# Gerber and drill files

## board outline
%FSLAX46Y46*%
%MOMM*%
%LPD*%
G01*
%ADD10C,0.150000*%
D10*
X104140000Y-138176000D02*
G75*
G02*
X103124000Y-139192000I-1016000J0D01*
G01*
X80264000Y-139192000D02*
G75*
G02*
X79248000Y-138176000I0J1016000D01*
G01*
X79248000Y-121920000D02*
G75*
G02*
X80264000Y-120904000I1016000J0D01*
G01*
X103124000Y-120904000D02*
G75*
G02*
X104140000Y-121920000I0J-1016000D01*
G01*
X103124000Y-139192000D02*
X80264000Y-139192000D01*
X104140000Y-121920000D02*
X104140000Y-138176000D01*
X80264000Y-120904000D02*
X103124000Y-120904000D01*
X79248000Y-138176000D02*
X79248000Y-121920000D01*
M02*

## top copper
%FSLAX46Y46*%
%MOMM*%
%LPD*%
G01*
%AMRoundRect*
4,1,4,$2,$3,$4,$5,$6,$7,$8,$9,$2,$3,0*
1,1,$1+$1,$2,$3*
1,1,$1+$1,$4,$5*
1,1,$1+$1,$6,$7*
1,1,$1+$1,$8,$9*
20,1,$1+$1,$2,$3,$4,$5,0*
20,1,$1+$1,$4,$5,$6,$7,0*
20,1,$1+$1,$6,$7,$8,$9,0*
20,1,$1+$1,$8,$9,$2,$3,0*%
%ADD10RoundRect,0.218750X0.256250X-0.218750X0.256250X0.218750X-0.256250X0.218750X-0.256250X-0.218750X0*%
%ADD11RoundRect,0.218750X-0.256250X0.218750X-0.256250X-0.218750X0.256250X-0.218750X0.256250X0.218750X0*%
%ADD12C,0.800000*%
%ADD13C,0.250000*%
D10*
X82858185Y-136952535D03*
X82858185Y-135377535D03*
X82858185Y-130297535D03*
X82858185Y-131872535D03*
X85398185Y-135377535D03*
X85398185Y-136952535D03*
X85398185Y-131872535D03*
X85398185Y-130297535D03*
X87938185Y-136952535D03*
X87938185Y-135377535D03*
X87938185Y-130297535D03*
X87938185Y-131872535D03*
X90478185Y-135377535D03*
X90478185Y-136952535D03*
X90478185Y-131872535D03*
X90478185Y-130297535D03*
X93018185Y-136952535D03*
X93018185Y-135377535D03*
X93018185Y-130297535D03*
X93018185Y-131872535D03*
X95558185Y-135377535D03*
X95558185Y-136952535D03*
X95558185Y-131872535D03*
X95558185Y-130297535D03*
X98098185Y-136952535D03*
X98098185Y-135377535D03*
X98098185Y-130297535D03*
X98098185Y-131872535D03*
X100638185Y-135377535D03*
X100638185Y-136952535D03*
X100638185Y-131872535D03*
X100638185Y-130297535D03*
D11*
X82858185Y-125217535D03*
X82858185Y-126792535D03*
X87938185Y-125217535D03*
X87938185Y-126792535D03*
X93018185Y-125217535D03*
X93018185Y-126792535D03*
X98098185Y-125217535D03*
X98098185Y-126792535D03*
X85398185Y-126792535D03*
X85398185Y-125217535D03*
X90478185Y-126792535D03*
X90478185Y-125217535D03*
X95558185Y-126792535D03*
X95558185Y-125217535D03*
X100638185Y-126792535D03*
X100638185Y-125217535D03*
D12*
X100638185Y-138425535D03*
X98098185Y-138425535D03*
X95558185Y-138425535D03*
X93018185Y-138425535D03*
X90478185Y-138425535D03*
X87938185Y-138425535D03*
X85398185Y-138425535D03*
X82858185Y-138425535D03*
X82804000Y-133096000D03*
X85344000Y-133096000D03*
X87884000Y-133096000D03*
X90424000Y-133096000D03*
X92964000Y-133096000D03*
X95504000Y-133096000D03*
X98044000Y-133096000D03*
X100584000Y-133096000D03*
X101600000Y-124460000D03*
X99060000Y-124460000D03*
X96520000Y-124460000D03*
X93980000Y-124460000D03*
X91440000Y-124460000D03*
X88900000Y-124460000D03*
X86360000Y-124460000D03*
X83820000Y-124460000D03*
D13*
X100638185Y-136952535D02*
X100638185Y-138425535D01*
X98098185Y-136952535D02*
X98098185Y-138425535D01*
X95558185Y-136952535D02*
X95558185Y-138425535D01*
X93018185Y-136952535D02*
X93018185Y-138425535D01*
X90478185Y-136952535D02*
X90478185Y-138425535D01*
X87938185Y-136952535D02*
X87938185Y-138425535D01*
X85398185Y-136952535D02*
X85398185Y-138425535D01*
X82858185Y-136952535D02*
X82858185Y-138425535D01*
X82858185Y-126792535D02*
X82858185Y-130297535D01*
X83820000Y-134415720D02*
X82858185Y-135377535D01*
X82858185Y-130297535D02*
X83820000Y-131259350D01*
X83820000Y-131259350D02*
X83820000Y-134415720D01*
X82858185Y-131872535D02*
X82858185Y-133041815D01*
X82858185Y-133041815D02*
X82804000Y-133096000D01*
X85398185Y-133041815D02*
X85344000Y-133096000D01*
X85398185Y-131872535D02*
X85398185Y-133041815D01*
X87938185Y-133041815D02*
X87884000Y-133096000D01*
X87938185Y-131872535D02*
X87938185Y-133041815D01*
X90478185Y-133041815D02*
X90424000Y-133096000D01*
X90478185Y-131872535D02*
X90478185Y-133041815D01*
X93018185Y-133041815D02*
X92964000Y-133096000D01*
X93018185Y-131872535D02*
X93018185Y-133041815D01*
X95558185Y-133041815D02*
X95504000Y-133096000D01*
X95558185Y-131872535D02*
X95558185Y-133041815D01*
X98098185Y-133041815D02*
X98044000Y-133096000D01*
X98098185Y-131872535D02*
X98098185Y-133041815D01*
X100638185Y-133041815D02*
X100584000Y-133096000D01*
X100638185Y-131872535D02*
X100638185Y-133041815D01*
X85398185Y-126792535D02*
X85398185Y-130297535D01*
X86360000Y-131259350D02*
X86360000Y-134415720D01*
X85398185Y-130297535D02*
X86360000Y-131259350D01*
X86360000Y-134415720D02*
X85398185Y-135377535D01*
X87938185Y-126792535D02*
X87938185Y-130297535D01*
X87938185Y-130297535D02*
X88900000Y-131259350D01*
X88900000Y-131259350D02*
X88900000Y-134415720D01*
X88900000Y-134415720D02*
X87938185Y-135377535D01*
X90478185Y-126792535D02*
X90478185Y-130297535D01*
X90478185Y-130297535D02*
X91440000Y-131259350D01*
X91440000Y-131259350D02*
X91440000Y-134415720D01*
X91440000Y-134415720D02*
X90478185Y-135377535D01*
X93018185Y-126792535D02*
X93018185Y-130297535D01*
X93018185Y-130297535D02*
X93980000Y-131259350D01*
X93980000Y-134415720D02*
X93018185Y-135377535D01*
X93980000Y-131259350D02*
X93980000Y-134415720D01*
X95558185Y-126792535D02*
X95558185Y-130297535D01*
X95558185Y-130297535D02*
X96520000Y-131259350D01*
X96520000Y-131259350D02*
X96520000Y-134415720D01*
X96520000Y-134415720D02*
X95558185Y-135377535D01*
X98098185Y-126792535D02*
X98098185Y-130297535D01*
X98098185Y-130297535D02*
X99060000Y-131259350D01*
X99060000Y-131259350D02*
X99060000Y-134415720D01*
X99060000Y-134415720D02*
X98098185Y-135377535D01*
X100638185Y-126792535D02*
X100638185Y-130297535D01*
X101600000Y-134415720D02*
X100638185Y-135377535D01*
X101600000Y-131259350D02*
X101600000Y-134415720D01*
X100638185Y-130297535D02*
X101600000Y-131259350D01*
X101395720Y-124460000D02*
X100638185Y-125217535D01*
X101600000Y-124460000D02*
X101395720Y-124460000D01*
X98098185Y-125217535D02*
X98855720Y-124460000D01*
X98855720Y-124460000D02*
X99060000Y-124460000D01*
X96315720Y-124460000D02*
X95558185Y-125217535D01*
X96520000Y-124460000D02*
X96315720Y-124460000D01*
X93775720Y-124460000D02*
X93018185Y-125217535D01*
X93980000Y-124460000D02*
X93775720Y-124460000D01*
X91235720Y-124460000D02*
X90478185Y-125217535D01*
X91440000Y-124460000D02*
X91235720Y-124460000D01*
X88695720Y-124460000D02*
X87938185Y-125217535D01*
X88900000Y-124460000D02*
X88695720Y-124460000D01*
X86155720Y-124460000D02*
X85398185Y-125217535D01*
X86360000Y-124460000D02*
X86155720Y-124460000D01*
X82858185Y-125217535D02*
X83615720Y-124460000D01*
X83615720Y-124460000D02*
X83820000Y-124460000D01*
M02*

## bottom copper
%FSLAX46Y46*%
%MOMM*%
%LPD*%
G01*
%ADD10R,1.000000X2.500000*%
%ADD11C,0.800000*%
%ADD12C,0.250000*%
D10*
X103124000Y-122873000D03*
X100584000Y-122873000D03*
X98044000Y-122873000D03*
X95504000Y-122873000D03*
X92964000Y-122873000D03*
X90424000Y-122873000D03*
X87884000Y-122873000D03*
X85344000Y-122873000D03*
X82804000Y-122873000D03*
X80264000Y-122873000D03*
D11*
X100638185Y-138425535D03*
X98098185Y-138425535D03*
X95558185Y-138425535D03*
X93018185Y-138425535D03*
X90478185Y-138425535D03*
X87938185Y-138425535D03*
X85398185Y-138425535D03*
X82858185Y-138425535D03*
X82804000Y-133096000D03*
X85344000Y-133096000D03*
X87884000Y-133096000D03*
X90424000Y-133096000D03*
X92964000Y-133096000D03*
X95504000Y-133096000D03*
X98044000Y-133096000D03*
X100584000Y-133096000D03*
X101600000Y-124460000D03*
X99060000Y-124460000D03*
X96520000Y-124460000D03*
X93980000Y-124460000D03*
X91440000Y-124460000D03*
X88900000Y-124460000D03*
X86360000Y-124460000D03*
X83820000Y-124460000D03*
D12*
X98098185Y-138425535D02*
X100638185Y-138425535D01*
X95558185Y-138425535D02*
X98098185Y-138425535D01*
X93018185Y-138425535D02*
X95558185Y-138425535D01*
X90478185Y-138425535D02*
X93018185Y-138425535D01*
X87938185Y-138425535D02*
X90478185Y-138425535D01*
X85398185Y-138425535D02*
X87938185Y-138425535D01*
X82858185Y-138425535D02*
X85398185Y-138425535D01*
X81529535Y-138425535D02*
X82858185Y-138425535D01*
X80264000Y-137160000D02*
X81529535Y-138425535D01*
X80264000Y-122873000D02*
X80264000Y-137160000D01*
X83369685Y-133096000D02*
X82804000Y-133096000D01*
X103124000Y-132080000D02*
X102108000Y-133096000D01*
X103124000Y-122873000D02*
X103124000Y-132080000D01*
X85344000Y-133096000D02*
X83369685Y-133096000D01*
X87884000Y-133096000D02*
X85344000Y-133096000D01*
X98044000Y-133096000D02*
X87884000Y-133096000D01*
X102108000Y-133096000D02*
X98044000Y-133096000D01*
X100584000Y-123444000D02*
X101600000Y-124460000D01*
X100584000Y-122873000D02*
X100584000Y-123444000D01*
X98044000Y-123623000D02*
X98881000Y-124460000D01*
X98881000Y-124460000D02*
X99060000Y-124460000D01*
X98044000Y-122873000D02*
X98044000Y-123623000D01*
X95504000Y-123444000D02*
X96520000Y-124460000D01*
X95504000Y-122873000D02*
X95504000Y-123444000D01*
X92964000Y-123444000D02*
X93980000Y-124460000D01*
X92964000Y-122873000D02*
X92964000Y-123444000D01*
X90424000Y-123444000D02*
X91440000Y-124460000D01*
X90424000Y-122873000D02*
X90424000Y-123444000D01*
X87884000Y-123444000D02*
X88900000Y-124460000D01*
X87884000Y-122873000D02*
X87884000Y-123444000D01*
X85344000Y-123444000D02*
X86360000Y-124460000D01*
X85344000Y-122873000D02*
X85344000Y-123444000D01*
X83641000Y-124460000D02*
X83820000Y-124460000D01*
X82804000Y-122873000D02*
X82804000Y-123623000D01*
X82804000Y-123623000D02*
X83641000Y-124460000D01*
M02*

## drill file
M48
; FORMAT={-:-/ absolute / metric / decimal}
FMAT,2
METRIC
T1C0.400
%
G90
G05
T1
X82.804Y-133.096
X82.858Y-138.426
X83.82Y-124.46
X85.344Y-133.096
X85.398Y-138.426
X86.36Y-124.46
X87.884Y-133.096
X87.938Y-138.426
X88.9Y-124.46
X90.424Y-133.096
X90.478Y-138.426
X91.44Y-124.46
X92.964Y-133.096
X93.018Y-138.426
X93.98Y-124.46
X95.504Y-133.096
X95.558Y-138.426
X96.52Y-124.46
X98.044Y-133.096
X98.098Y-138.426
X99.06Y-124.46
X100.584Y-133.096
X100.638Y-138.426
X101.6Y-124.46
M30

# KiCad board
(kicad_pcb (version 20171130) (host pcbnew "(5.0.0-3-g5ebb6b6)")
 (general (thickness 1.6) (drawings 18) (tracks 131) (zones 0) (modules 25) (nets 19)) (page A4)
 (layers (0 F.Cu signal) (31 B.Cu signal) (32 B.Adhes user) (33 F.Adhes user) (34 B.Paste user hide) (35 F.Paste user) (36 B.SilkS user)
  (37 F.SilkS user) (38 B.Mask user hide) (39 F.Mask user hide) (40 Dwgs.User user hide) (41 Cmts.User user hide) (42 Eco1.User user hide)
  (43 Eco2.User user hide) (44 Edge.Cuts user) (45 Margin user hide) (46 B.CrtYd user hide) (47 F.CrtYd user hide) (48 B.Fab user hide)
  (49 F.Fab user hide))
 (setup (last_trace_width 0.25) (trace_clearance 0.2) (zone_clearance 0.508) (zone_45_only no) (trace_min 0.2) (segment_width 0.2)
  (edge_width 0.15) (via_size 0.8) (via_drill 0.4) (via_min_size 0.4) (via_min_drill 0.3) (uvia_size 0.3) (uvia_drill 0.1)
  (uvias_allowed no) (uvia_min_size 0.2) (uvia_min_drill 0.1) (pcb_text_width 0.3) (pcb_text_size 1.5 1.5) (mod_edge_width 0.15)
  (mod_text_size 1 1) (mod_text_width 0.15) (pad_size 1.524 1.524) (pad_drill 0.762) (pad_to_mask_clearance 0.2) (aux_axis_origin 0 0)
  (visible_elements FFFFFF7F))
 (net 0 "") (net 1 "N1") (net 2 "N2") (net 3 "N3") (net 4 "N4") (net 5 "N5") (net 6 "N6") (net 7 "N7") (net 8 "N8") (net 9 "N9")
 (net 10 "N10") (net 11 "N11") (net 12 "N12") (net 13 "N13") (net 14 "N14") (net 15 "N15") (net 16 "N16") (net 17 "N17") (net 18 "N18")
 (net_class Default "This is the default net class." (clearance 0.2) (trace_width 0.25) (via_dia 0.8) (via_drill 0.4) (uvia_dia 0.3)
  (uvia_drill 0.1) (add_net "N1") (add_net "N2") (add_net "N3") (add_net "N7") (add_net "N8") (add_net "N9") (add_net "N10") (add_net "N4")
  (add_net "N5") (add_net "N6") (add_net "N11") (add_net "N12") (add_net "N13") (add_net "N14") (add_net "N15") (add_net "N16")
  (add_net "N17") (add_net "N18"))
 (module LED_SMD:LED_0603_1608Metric (layer F.Cu) (at 82.858185 136.165035 90)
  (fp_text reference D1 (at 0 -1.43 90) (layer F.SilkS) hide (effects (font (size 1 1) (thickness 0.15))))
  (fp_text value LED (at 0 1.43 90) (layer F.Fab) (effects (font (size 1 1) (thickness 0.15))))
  (pad 1 smd roundrect (at -0.7875 0 90) (size 0.875 0.95) (layers F.Cu F.Paste F.Mask) (roundrect_rratio 0.25) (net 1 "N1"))
  (pad 2 smd roundrect (at 0.7875 0 90) (size 0.875 0.95) (layers F.Cu F.Paste F.Mask) (roundrect_rratio 0.25) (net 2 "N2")))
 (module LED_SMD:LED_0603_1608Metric (layer F.Cu) (at 82.858185 131.085035 90)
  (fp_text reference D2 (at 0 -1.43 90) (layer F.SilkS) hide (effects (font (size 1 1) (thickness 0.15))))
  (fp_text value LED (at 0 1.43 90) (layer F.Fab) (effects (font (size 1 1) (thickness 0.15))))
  (pad 2 smd roundrect (at 0.7875 0 90) (size 0.875 0.95) (layers F.Cu F.Paste F.Mask) (roundrect_rratio 0.25) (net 2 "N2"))
  (pad 1 smd roundrect (at -0.7875 0 90) (size 0.875 0.95) (layers F.Cu F.Paste F.Mask) (roundrect_rratio 0.25) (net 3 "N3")))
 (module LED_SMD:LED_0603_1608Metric (layer F.Cu) (at 85.398185 136.165035 90)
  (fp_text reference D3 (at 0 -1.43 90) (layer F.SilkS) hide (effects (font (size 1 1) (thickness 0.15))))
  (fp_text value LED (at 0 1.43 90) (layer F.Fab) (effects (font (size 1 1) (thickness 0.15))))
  (pad 2 smd roundrect (at 0.7875 0 90) (size 0.875 0.95) (layers F.Cu F.Paste F.Mask) (roundrect_rratio 0.25) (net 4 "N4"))
  (pad 1 smd roundrect (at -0.7875 0 90) (size 0.875 0.95) (layers F.Cu F.Paste F.Mask) (roundrect_rratio 0.25) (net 1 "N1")))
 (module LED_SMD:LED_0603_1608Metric (layer F.Cu) (at 85.398185 131.085035 90)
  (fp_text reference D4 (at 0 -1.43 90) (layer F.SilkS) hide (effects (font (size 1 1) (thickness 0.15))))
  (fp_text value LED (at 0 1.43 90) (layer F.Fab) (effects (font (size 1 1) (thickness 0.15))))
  (pad 1 smd roundrect (at -0.7875 0 90) (size 0.875 0.95) (layers F.Cu F.Paste F.Mask) (roundrect_rratio 0.25) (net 3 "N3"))
  (pad 2 smd roundrect (at 0.7875 0 90) (size 0.875 0.95) (layers F.Cu F.Paste F.Mask) (roundrect_rratio 0.25) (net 4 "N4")))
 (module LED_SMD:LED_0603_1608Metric (layer F.Cu) (at 87.938185 136.165035 90)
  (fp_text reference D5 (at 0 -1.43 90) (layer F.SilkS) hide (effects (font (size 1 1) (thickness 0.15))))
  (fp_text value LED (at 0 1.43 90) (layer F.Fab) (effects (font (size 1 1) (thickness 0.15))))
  (pad 1 smd roundrect (at -0.7875 0 90) (size 0.875 0.95) (layers F.Cu F.Paste F.Mask) (roundrect_rratio 0.25) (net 1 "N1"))
  (pad 2 smd roundrect (at 0.7875 0 90) (size 0.875 0.95) (layers F.Cu F.Paste F.Mask) (roundrect_rratio 0.25) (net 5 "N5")))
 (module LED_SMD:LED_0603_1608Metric (layer F.Cu) (at 87.938185 131.085035 90)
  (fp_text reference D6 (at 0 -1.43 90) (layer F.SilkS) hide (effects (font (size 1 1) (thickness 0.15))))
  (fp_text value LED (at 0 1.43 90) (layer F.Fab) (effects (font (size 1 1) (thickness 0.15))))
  (pad 2 smd roundrect (at 0.7875 0 90) (size 0.875 0.95) (layers F.Cu F.Paste F.Mask) (roundrect_rratio 0.25) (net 5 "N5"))
  (pad 1 smd roundrect (at -0.7875 0 90) (size 0.875 0.95) (layers F.Cu F.Paste F.Mask) (roundrect_rratio 0.25) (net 3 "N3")))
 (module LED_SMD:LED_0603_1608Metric (layer F.Cu) (at 90.478185 136.165035 90)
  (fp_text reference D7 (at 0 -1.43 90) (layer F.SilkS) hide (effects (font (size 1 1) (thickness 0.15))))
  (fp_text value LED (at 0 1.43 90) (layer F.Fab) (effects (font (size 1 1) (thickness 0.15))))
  (pad 2 smd roundrect (at 0.7875 0 90) (size 0.875 0.95) (layers F.Cu F.Paste F.Mask) (roundrect_rratio 0.25) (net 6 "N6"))
  (pad 1 smd roundrect (at -0.7875 0 90) (size 0.875 0.95) (layers F.Cu F.Paste F.Mask) (roundrect_rratio 0.25) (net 1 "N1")))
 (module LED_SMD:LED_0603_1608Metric (layer F.Cu) (at 90.478185 131.085035 90)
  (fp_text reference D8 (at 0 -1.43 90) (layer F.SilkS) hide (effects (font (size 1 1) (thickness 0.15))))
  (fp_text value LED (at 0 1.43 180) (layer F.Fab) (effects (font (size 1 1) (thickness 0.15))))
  (pad 1 smd roundrect (at -0.7875 0 90) (size 0.875 0.95) (layers F.Cu F.Paste F.Mask) (roundrect_rratio 0.25) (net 3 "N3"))
  (pad 2 smd roundrect (at 0.7875 0 90) (size 0.875 0.95) (layers F.Cu F.Paste F.Mask) (roundrect_rratio 0.25) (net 6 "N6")))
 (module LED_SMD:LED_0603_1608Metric (layer F.Cu) (at 93.018185 136.165035 90)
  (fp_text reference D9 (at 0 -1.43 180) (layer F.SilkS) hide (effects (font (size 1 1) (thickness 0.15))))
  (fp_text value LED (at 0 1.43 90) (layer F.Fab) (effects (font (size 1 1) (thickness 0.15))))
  (pad 1 smd roundrect (at -0.7875 0 90) (size 0.875 0.95) (layers F.Cu F.Paste F.Mask) (roundrect_rratio 0.25) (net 1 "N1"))
  (pad 2 smd roundrect (at 0.7875 0 90) (size 0.875 0.95) (layers F.Cu F.Paste F.Mask) (roundrect_rratio 0.25) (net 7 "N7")))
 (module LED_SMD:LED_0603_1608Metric (layer F.Cu) (at 93.018185 131.085035 90)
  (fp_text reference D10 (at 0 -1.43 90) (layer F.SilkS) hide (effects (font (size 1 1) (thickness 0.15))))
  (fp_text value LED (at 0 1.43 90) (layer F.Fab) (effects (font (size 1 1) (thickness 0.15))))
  (pad 2 smd roundrect (at 0.7875 0 90) (size 0.875 0.95) (layers F.Cu F.Paste F.Mask) (roundrect_rratio 0.25) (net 7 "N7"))
  (pad 1 smd roundrect (at -0.7875 0 90) (size 0.875 0.95) (layers F.Cu F.Paste F.Mask) (roundrect_rratio 0.25) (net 3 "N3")))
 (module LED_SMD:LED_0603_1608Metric (layer F.Cu) (at 95.558185 136.165035 90)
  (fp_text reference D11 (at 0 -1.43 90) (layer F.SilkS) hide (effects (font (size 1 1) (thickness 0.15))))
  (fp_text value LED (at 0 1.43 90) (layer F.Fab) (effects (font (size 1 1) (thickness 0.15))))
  (pad 2 smd roundrect (at 0.7875 0 90) (size 0.875 0.95) (layers F.Cu F.Paste F.Mask) (roundrect_rratio 0.25) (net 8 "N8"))
  (pad 1 smd roundrect (at -0.7875 0 90) (size 0.875 0.95) (layers F.Cu F.Paste F.Mask) (roundrect_rratio 0.25) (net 1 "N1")))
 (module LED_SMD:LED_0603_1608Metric (layer F.Cu) (at 95.558185 131.085035 90)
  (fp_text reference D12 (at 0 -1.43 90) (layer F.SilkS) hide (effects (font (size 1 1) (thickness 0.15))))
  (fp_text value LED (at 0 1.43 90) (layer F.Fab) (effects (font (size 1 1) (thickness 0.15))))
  (pad 1 smd roundrect (at -0.7875 0 90) (size 0.875 0.95) (layers F.Cu F.Paste F.Mask) (roundrect_rratio 0.25) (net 3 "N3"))
  (pad 2 smd roundrect (at 0.7875 0 90) (size 0.875 0.95) (layers F.Cu F.Paste F.Mask) (roundrect_rratio 0.25) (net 8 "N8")))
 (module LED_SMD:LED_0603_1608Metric (layer F.Cu) (at 98.098185 136.165035 90)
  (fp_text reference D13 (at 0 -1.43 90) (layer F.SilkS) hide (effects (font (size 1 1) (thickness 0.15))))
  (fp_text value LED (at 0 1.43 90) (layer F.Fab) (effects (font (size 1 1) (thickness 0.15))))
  (pad 1 smd roundrect (at -0.7875 0 90) (size 0.875 0.95) (layers F.Cu F.Paste F.Mask) (roundrect_rratio 0.25) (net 1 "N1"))
  (pad 2 smd roundrect (at 0.7875 0 90) (size 0.875 0.95) (layers F.Cu F.Paste F.Mask) (roundrect_rratio 0.25) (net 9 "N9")))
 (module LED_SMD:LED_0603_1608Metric (layer F.Cu) (at 98.098185 131.085035 90)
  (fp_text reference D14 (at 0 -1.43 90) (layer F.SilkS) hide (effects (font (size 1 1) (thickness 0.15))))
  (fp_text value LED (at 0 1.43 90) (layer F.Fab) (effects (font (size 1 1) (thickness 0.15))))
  (pad 2 smd roundrect (at 0.7875 0 90) (size 0.875 0.95) (layers F.Cu F.Paste F.Mask) (roundrect_rratio 0.25) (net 9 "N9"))
  (pad 1 smd roundrect (at -0.7875 0 90) (size 0.875 0.95) (layers F.Cu F.Paste F.Mask) (roundrect_rratio 0.25) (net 3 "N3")))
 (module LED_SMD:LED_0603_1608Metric (layer F.Cu) (at 100.638185 136.165035 90)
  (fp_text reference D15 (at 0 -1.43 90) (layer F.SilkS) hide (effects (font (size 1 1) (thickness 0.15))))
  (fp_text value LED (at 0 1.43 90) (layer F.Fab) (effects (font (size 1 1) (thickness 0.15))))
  (pad 2 smd roundrect (at 0.7875 0 90) (size 0.875 0.95) (layers F.Cu F.Paste F.Mask) (roundrect_rratio 0.25) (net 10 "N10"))
  (pad 1 smd roundrect (at -0.7875 0 90) (size 0.875 0.95) (layers F.Cu F.Paste F.Mask) (roundrect_rratio 0.25) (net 1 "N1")))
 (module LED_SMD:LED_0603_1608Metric (layer F.Cu) (at 100.638185 131.085035 90)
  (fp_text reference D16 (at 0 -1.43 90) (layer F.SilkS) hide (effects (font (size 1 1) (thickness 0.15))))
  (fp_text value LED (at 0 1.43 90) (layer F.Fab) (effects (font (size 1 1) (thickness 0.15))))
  (pad 1 smd roundrect (at -0.7875 0 90) (size 0.875 0.95) (layers F.Cu F.Paste F.Mask) (roundrect_rratio 0.25) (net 3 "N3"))
  (pad 2 smd roundrect (at 0.7875 0 90) (size 0.875 0.95) (layers F.Cu F.Paste F.Mask) (roundrect_rratio 0.25) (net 10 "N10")))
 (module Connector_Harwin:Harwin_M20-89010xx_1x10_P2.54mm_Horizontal (layer B.Cu) (at 91.694 117.348 90)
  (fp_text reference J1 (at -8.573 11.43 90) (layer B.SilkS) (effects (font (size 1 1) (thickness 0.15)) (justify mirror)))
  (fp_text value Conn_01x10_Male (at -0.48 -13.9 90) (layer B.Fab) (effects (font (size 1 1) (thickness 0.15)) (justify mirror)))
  (pad 1 smd rect (at -5.525 11.43 90) (size 2.5 1) (layers B.Cu B.Paste B.Mask) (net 3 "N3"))
  (pad 2 smd rect (at -5.525 8.89 90) (size 2.5 1) (layers B.Cu B.Paste B.Mask) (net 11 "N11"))
  (pad 3 smd rect (at -5.525 6.35 90) (size 2.5 1) (layers B.Cu B.Paste B.Mask) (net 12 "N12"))
  (pad 4 smd rect (at -5.525 3.81 90) (size 2.5 1) (layers B.Cu B.Paste B.Mask) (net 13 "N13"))
  (pad 5 smd rect (at -5.525 1.27 90) (size 2.5 1) (layers B.Cu B.Paste B.Mask) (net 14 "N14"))
  (pad 6 smd rect (at -5.525 -1.27 90) (size 2.5 1) (layers B.Cu B.Paste B.Mask) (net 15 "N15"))
  (pad 7 smd rect (at -5.525 -3.81 90) (size 2.5 1) (layers B.Cu B.Paste B.Mask) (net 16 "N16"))
  (pad 8 smd rect (at -5.525 -6.35 90) (size 2.5 1) (layers B.Cu B.Paste B.Mask) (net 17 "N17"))
  (pad 9 smd rect (at -5.525 -8.89 90) (size 2.5 1) (layers B.Cu B.Paste B.Mask) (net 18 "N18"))
  (pad 10 smd rect (at -5.525 -11.43 90) (size 2.5 1) (layers B.Cu B.Paste B.Mask) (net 1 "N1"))
  (pad "" smd rect (at 3.895 11.43 90) (size 6 0.76) (layers B.SilkS)))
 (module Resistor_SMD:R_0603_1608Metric (layer F.Cu) (at 82.858185 126.005035 270)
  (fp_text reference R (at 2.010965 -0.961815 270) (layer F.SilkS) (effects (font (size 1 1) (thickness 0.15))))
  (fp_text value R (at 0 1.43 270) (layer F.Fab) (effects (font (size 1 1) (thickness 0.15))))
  (pad 1 smd roundrect (at -0.7875 0 270) (size 0.875 0.95) (layers F.Cu F.Paste F.Mask) (roundrect_rratio 0.25) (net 18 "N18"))
  (pad 2 smd roundrect (at 0.7875 0 270) (size 0.875 0.95) (layers F.Cu F.Paste F.Mask) (roundrect_rratio 0.25) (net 2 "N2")))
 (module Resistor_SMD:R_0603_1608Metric (layer F.Cu) (at 87.938185 126.005035 270)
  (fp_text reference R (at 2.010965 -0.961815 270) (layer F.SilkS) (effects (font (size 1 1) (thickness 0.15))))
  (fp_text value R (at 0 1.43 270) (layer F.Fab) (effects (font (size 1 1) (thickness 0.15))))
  (pad 1 smd roundrect (at -0.7875 0 270) (size 0.875 0.95) (layers F.Cu F.Paste F.Mask) (roundrect_rratio 0.25) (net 16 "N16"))
  (pad 2 smd roundrect (at 0.7875 0 270) (size 0.875 0.95) (layers F.Cu F.Paste F.Mask) (roundrect_rratio 0.25) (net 5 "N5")))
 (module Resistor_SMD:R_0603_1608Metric (layer F.Cu) (at 93.018185 126.005035 270)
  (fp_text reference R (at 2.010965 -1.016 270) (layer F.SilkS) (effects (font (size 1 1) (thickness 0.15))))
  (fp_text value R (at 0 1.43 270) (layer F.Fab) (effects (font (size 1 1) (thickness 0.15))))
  (pad 1 smd roundrect (at -0.7875 0 270) (size 0.875 0.95) (layers F.Cu F.Paste F.Mask) (roundrect_rratio 0.25) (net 14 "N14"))
  (pad 2 smd roundrect (at 0.7875 0 270) (size 0.875 0.95) (layers F.Cu F.Paste F.Mask) (roundrect_rratio 0.25) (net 7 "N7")))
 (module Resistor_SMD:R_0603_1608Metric (layer F.Cu) (at 98.098185 126.005035 270)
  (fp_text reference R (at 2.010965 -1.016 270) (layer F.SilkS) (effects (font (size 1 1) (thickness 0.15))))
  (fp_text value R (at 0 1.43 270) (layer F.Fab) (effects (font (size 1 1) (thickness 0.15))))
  (pad 1 smd roundrect (at -0.7875 0 270) (size 0.875 0.95) (layers F.Cu F.Paste F.Mask) (roundrect_rratio 0.25) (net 12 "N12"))
  (pad 2 smd roundrect (at 0.7875 0 270) (size 0.875 0.95) (layers F.Cu F.Paste F.Mask) (roundrect_rratio 0.25) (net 9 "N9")))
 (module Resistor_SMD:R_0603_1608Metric (layer F.Cu) (at 85.398185 126.005035 270)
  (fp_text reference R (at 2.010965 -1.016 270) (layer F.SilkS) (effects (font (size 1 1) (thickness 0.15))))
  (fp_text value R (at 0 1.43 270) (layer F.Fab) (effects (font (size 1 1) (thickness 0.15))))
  (pad 2 smd roundrect (at 0.7875 0 270) (size 0.875 0.95) (layers F.Cu F.Paste F.Mask) (roundrect_rratio 0.25) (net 4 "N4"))
  (pad 1 smd roundrect (at -0.7875 0 270) (size 0.875 0.95) (layers F.Cu F.Paste F.Mask) (roundrect_rratio 0.25) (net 17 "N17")))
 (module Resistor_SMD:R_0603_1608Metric (layer F.Cu) (at 90.478185 126.005035 270)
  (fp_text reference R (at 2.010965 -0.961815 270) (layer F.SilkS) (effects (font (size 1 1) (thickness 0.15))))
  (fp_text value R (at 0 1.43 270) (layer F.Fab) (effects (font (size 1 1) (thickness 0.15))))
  (pad 2 smd roundrect (at 0.7875 0 270) (size 0.875 0.95) (layers F.Cu F.Paste F.Mask) (roundrect_rratio 0.25) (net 6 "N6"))
  (pad 1 smd roundrect (at -0.7875 0 270) (size 0.875 0.95) (layers F.Cu F.Paste F.Mask) (roundrect_rratio 0.25) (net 15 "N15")))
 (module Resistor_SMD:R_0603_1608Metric (layer F.Cu) (at 95.558185 126.005035 270)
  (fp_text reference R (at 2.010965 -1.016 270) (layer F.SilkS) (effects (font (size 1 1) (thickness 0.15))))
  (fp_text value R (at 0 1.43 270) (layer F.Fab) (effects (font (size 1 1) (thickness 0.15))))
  (pad 2 smd roundrect (at 0.7875 0 270) (size 0.875 0.95) (layers F.Cu F.Paste F.Mask) (roundrect_rratio 0.25) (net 8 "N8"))
  (pad 1 smd roundrect (at -0.7875 0 270) (size 0.875 0.95) (layers F.Cu F.Paste F.Mask) (roundrect_rratio 0.25) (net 13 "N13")))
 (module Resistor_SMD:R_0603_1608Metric (layer F.Cu) (at 100.638185 126.005035 270)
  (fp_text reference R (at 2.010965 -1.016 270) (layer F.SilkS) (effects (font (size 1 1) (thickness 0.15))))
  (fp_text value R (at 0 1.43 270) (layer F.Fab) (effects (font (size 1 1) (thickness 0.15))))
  (pad 2 smd roundrect (at 0.7875 0 270) (size 0.875 0.95) (layers F.Cu F.Paste F.Mask) (roundrect_rratio 0.25) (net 10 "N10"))
  (pad 1 smd roundrect (at -0.7875 0 270) (size 0.875 0.95) (layers F.Cu F.Paste F.Mask) (roundrect_rratio 0.25) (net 11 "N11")))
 (gr_arc (start 103.124 138.176) (end 103.124 139.192) (angle -90) (layer Edge.Cuts) (width 0.15))
 (gr_arc (start 80.264 138.176) (end 79.248 138.176) (angle -90) (layer Edge.Cuts) (width 0.15))
 (gr_arc (start 80.264 121.92) (end 80.264 120.904) (angle -90) (layer Edge.Cuts) (width 0.15))
 (gr_arc (start 103.124 121.92) (end 104.14 121.92) (angle -90) (layer Edge.Cuts) (width 0.15))
 (gr_line (start 103.124 139.192) (end 80.264 139.192) (layer Edge.Cuts) (width 0.15))
 (gr_line (start 104.14 121.92) (end 104.14 138.176) (layer Edge.Cuts) (width 0.15))
 (gr_line (start 80.264 120.904) (end 103.124 120.904) (layer Edge.Cuts) (width 0.15))
 (gr_line (start 79.248 138.176) (end 79.248 121.92) (layer Edge.Cuts) (width 0.15))
 (via (at 100.638185 138.425535) (size 0.8) (drill 0.4) (layers F.Cu B.Cu) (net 1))
 (segment (start 100.638185 136.952535) (end 100.638185 138.425535) (width 0.25) (layer F.Cu) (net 1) (status 10))
 (via (at 98.098185 138.425535) (size 0.8) (drill 0.4) (layers F.Cu B.Cu) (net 1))
 (segment (start 98.098185 136.952535) (end 98.098185 138.425535) (width 0.25) (layer F.Cu) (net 1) (status 10))
 (segment (start 98.098185 138.425535) (end 100.638185 138.425535) (width 0.25) (layer B.Cu) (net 1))
 (via (at 95.558185 138.425535) (size 0.8) (drill 0.4) (layers F.Cu B.Cu) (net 1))
 (segment (start 95.558185 136.952535) (end 95.558185 138.425535) (width 0.25) (layer F.Cu) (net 1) (status 10))
 (segment (start 95.558185 138.425535) (end 98.098185 138.425535) (width 0.25) (layer B.Cu) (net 1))
 (via (at 93.018185 138.425535) (size 0.8) (drill 0.4) (layers F.Cu B.Cu) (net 1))
 (segment (start 93.018185 136.952535) (end 93.018185 138.425535) (width 0.25) (layer F.Cu) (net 1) (status 10))
 (segment (start 93.018185 138.425535) (end 95.558185 138.425535) (width 0.25) (layer B.Cu) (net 1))
 (via (at 90.478185 138.425535) (size 0.8) (drill 0.4) (layers F.Cu B.Cu) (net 1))
 (segment (start 90.478185 136.952535) (end 90.478185 138.425535) (width 0.25) (layer F.Cu) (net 1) (status 10))
 (segment (start 90.478185 138.425535) (end 93.018185 138.425535) (width 0.25) (layer B.Cu) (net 1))
 (segment (start 87.938185 136.952535) (end 87.938185 138.425535) (width 0.25) (layer F.Cu) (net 1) (status 10))
 (segment (start 87.938185 138.425535) (end 90.478185 138.425535) (width 0.25) (layer B.Cu) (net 1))
 (via (at 87.938185 138.425535) (size 0.8) (drill 0.4) (layers F.Cu B.Cu) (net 1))
 (segment (start 85.398185 138.425535) (end 87.938185 138.425535) (width 0.25) (layer B.Cu) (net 1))
 (via (at 85.398185 138.425535) (size 0.8) (drill 0.4) (layers F.Cu B.Cu) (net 1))
 (segment (start 85.398185 136.952535) (end 85.398185 138.425535) (width 0.25) (layer F.Cu) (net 1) (status 10))
 (via (at 82.858185 138.425535) (size 0.8) (drill 0.4) (layers F.Cu B.Cu) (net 1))
 (segment (start 82.858185 136.952535) (end 82.858185 138.425535) (width 0.25) (layer F.Cu) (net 1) (status 10))
 (segment (start 82.858185 138.425535) (end 85.398185 138.425535) (width 0.25) (layer B.Cu) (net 1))
 (segment (start 81.529535 138.425535) (end 82.858185 138.425535) (width 0.25) (layer B.Cu) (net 1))
 (segment (start 80.264 137.16) (end 81.529535 138.425535) (width 0.25) (layer B.Cu) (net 1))
 (segment (start 80.264 122.873) (end 80.264 137.16) (width 0.25) (layer B.Cu) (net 1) (status 10))
 (segment (start 82.858185 126.792535) (end 82.858185 130.297535) (width 0.25) (layer F.Cu) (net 2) (status 30))
 (segment (start 83.82 134.41572) (end 82.858185 135.377535) (width 0.25) (layer F.Cu) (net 2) (status 20))
 (segment (start 82.858185 130.297535) (end 83.82 131.25935) (width 0.25) (layer F.Cu) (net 2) (status 10))
 (segment (start 83.82 131.25935) (end 83.82 134.41572) (width 0.25) (layer F.Cu) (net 2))
 (via (at 82.804 133.096) (size 0.8) (drill 0.4) (layers F.Cu B.Cu) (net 3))
 (segment (start 82.858185 131.872535) (end 82.858185 133.041815) (width 0.25) (layer F.Cu) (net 3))
 (segment (start 82.858185 133.041815) (end 82.804 133.096) (width 0.25) (layer F.Cu) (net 3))
 (segment (start 83.369685 133.096) (end 82.804 133.096) (width 0.25) (layer B.Cu) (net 3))
 (segment (start 103.124 132.08) (end 102.108 133.096) (width 0.25) (layer B.Cu) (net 3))
 (segment (start 103.124 122.873) (end 103.124 132.08) (width 0.25) (layer B.Cu) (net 3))
 (via (at 85.344 133.096) (size 0.8) (drill 0.4) (layers F.Cu B.Cu) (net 3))
 (segment (start 85.398185 133.041815) (end 85.344 133.096) (width 0.25) (layer F.Cu) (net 3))
 (segment (start 85.398185 131.872535) (end 85.398185 133.041815) (width 0.25) (layer F.Cu) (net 3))
 (segment (start 85.344 133.096) (end 83.369685 133.096) (width 0.25) (layer B.Cu) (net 3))
 (segment (start 87.938185 133.041815) (end 87.884 133.096) (width 0.25) (layer F.Cu) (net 3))
 (segment (start 87.938185 131.872535) (end 87.938185 133.041815) (width 0.25) (layer F.Cu) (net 3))
 (via (at 87.884 133.096) (size 0.8) (drill 0.4) (layers F.Cu B.Cu) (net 3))
 (segment (start 87.884 133.096) (end 85.344 133.096) (width 0.25) (layer B.Cu) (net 3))
 (via (at 90.424 133.096) (size 0.8) (drill 0.4) (layers F.Cu B.Cu) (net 3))
 (segment (start 90.478185 133.041815) (end 90.424 133.096) (width 0.25) (layer F.Cu) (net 3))
 (segment (start 90.478185 131.872535) (end 90.478185 133.041815) (width 0.25) (layer F.Cu) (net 3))
 (segment (start 93.018185 133.041815) (end 92.964 133.096) (width 0.25) (layer F.Cu) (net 3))
 (via (at 92.964 133.096) (size 0.8) (drill 0.4) (layers F.Cu B.Cu) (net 3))
 (segment (start 93.018185 131.872535) (end 93.018185 133.041815) (width 0.25) (layer F.Cu) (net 3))
 (via (at 95.504 133.096) (size 0.8) (drill 0.4) (layers F.Cu B.Cu) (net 3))
 (segment (start 95.558185 133.041815) (end 95.504 133.096) (width 0.25) (layer F.Cu) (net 3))
 (segment (start 95.558185 131.872535) (end 95.558185 133.041815) (width 0.25) (layer F.Cu) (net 3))
 (segment (start 98.098185 133.041815) (end 98.044 133.096) (width 0.25) (layer F.Cu) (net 3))
 (segment (start 98.098185 131.872535) (end 98.098185 133.041815) (width 0.25) (layer F.Cu) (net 3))
 (segment (start 98.044 133.096) (end 87.884 133.096) (width 0.25) (layer B.Cu) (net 3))
 (via (at 98.044 133.096) (size 0.8) (drill 0.4) (layers F.Cu B.Cu) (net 3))
 (segment (start 102.108 133.096) (end 98.044 133.096) (width 0.25) (layer B.Cu) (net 3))
 (via (at 100.584 133.096) (size 0.8) (drill 0.4) (layers F.Cu B.Cu) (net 3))
 (segment (start 100.638185 133.041815) (end 100.584 133.096) (width 0.25) (layer F.Cu) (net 3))
 (segment (start 100.638185 131.872535) (end 100.638185 133.041815) (width 0.25) (layer F.Cu) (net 3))
 (segment (start 85.398185 126.792535) (end 85.398185 130.297535) (width 0.25) (layer F.Cu) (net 4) (status 30))
 (segment (start 86.36 131.25935) (end 86.36 134.41572) (width 0.25) (layer F.Cu) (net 4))
 (segment (start 85.398185 130.297535) (end 86.36 131.25935) (width 0.25) (layer F.Cu) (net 4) (status 10))
 (segment (start 86.36 134.41572) (end 85.398185 135.377535) (width 0.25) (layer F.Cu) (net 4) (status 20))
 (segment (start 87.938185 126.792535) (end 87.938185 130.297535) (width 0.25) (layer F.Cu) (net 5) (status 30))
 (segment (start 87.938185 130.297535) (end 88.9 131.25935) (width 0.25) (layer F.Cu) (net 5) (status 10))
 (segment (start 88.9 131.25935) (end 88.9 134.41572) (width 0.25) (layer F.Cu) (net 5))
 (segment (start 88.9 134.41572) (end 87.938185 135.377535) (width 0.25) (layer F.Cu) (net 5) (status 20))
 (segment (start 90.478185 126.792535) (end 90.478185 130.297535) (width 0.25) (layer F.Cu) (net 6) (status 30))
 (segment (start 90.478185 130.297535) (end 91.44 131.25935) (width 0.25) (layer F.Cu) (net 6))
 (segment (start 91.44 131.25935) (end 91.44 134.41572) (width 0.25) (layer F.Cu) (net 6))
 (segment (start 91.44 134.41572) (end 90.478185 135.377535) (width 0.25) (layer F.Cu) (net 6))
 (segment (start 93.018185 126.792535) (end 93.018185 130.297535) (width 0.25) (layer F.Cu) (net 7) (status 30))
 (segment (start 93.018185 130.297535) (end 93.98 131.25935) (width 0.25) (layer F.Cu) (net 7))
 (segment (start 93.98 134.41572) (end 93.018185 135.377535) (width 0.25) (layer F.Cu) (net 7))
 (segment (start 93.98 131.25935) (end 93.98 134.41572) (width 0.25) (layer F.Cu) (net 7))
 (segment (start 95.558185 126.792535) (end 95.558185 130.297535) (width 0.25) (layer F.Cu) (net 8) (status 30))
 (segment (start 95.558185 130.297535) (end 96.52 131.25935) (width 0.25) (layer F.Cu) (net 8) (status 10))
 (segment (start 96.52 131.25935) (end 96.52 134.41572) (width 0.25) (layer F.Cu) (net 8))
 (segment (start 96.52 134.41572) (end 95.558185 135.377535) (width 0.25) (layer F.Cu) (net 8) (status 20))
 (segment (start 98.098185 126.792535) (end 98.098185 130.297535) (width 0.25) (layer F.Cu) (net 9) (status 30))
 (segment (start 98.098185 130.297535) (end 99.06 131.25935) (width 0.25) (layer F.Cu) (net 9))
 (segment (start 99.06 131.25935) (end 99.06 134.41572) (width 0.25) (layer F.Cu) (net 9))
 (segment (start 99.06 134.41572) (end 98.098185 135.377535) (width 0.25) (layer F.Cu) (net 9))
 (segment (start 100.638185 126.792535) (end 100.638185 130.297535) (width 0.25) (layer F.Cu) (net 10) (status 30))
 (segment (start 101.6 134.41572) (end 100.638185 135.377535) (width 0.25) (layer F.Cu) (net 10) (status 20))
 (segment (start 101.6 131.25935) (end 101.6 134.41572) (width 0.25) (layer F.Cu) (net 10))
 (segment (start 100.638185 130.297535) (end 101.6 131.25935) (width 0.25) (layer F.Cu) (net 10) (status 10))
 (via (at 101.6 124.46) (size 0.8) (drill 0.4) (layers F.Cu B.Cu) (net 11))
 (segment (start 100.584 123.444) (end 101.6 124.46) (width 0.25) (layer B.Cu) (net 11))
 (segment (start 100.584 122.873) (end 100.584 123.444) (width 0.25) (layer B.Cu) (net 11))
 (segment (start 101.39572 124.46) (end 100.638185 125.217535) (width 0.25) (layer F.Cu) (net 11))
 (segment (start 101.6 124.46) (end 101.39572 124.46) (width 0.25) (layer F.Cu) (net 11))
 (segment (start 98.044 123.623) (end 98.881 124.46) (width 0.25) (layer B.Cu) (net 12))
 (segment (start 98.881 124.46) (end 99.06 124.46) (width 0.25) (layer B.Cu) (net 12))
 (via (at 99.06 124.46) (size 0.8) (drill 0.4) (layers F.Cu B.Cu) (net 12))
 (segment (start 98.044 122.873) (end 98.044 123.623) (width 0.25) (layer B.Cu) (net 12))
 (segment (start 98.098185 125.217535) (end 98.85572 124.46) (width 0.25) (layer F.Cu) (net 12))
 (segment (start 98.85572 124.46) (end 99.06 124.46) (width 0.25) (layer F.Cu) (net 12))
 (via (at 96.52 124.46) (size 0.8) (drill 0.4) (layers F.Cu B.Cu) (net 13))
 (segment (start 95.504 123.444) (end 96.52 124.46) (width 0.25) (layer B.Cu) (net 13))
 (segment (start 95.504 122.873) (end 95.504 123.444) (width 0.25) (layer B.Cu) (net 13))
 (segment (start 96.31572 124.46) (end 95.558185 125.217535) (width 0.25) (layer F.Cu) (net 13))
 (segment (start 96.52 124.46) (end 96.31572 124.46) (width 0.25) (layer F.Cu) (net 13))
 (via (at 93.98 124.46) (size 0.8) (drill 0.4) (layers F.Cu B.Cu) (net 14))
 (segment (start 92.964 123.444) (end 93.98 124.46) (width 0.25) (layer B.Cu) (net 14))
 (segment (start 92.964 122.873) (end 92.964 123.444) (width 0.25) (layer B.Cu) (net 14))
 (segment (start 93.77572 124.46) (end 93.018185 125.217535) (width 0.25) (layer F.Cu) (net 14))
 (segment (start 93.98 124.46) (end 93.77572 124.46) (width 0.25) (layer F.Cu) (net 14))
 (via (at 91.44 124.46) (size 0.8) (drill 0.4) (layers F.Cu B.Cu) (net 15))
 (segment (start 90.424 123.444) (end 91.44 124.46) (width 0.25) (layer B.Cu) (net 15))
 (segment (start 90.424 122.873) (end 90.424 123.444) (width 0.25) (layer B.Cu) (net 15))
 (segment (start 91.23572 124.46) (end 90.478185 125.217535) (width 0.25) (layer F.Cu) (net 15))
 (segment (start 91.44 124.46) (end 91.23572 124.46) (width 0.25) (layer F.Cu) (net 15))
 (via (at 88.9 124.46) (size 0.8) (drill 0.4) (layers F.Cu B.Cu) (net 16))
 (segment (start 87.884 123.444) (end 88.9 124.46) (width 0.25) (layer B.Cu) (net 16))
 (segment (start 87.884 122.873) (end 87.884 123.444) (width 0.25) (layer B.Cu) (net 16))
 (segment (start 88.69572 124.46) (end 87.938185 125.217535) (width 0.25) (layer F.Cu) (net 16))
 (segment (start 88.9 124.46) (end 88.69572 124.46) (width 0.25) (layer F.Cu) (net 16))
 (via (at 86.36 124.46) (size 0.8) (drill 0.4) (layers F.Cu B.Cu) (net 17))
 (segment (start 85.344 123.444) (end 86.36 124.46) (width 0.25) (layer B.Cu) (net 17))
 (segment (start 85.344 122.873) (end 85.344 123.444) (width 0.25) (layer B.Cu) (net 17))
 (segment (start 86.15572 124.46) (end 85.398185 125.217535) (width 0.25) (layer F.Cu) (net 17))
 (segment (start 86.36 124.46) (end 86.15572 124.46) (width 0.25) (layer F.Cu) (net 17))
 (via (at 83.82 124.46) (size 0.8) (drill 0.4) (layers F.Cu B.Cu) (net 18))
 (segment (start 83.641 124.46) (end 83.82 124.46) (width 0.25) (layer B.Cu) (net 18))
 (segment (start 82.804 122.873) (end 82.804 123.623) (width 0.25) (layer B.Cu) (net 18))
 (segment (start 82.804 123.623) (end 83.641 124.46) (width 0.25) (layer B.Cu) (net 18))
 (segment (start 82.858185 125.217535) (end 83.61572 124.46) (width 0.25) (layer F.Cu) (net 18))
 (segment (start 83.61572 124.46) (end 83.82 124.46) (width 0.25) (layer F.Cu) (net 18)))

